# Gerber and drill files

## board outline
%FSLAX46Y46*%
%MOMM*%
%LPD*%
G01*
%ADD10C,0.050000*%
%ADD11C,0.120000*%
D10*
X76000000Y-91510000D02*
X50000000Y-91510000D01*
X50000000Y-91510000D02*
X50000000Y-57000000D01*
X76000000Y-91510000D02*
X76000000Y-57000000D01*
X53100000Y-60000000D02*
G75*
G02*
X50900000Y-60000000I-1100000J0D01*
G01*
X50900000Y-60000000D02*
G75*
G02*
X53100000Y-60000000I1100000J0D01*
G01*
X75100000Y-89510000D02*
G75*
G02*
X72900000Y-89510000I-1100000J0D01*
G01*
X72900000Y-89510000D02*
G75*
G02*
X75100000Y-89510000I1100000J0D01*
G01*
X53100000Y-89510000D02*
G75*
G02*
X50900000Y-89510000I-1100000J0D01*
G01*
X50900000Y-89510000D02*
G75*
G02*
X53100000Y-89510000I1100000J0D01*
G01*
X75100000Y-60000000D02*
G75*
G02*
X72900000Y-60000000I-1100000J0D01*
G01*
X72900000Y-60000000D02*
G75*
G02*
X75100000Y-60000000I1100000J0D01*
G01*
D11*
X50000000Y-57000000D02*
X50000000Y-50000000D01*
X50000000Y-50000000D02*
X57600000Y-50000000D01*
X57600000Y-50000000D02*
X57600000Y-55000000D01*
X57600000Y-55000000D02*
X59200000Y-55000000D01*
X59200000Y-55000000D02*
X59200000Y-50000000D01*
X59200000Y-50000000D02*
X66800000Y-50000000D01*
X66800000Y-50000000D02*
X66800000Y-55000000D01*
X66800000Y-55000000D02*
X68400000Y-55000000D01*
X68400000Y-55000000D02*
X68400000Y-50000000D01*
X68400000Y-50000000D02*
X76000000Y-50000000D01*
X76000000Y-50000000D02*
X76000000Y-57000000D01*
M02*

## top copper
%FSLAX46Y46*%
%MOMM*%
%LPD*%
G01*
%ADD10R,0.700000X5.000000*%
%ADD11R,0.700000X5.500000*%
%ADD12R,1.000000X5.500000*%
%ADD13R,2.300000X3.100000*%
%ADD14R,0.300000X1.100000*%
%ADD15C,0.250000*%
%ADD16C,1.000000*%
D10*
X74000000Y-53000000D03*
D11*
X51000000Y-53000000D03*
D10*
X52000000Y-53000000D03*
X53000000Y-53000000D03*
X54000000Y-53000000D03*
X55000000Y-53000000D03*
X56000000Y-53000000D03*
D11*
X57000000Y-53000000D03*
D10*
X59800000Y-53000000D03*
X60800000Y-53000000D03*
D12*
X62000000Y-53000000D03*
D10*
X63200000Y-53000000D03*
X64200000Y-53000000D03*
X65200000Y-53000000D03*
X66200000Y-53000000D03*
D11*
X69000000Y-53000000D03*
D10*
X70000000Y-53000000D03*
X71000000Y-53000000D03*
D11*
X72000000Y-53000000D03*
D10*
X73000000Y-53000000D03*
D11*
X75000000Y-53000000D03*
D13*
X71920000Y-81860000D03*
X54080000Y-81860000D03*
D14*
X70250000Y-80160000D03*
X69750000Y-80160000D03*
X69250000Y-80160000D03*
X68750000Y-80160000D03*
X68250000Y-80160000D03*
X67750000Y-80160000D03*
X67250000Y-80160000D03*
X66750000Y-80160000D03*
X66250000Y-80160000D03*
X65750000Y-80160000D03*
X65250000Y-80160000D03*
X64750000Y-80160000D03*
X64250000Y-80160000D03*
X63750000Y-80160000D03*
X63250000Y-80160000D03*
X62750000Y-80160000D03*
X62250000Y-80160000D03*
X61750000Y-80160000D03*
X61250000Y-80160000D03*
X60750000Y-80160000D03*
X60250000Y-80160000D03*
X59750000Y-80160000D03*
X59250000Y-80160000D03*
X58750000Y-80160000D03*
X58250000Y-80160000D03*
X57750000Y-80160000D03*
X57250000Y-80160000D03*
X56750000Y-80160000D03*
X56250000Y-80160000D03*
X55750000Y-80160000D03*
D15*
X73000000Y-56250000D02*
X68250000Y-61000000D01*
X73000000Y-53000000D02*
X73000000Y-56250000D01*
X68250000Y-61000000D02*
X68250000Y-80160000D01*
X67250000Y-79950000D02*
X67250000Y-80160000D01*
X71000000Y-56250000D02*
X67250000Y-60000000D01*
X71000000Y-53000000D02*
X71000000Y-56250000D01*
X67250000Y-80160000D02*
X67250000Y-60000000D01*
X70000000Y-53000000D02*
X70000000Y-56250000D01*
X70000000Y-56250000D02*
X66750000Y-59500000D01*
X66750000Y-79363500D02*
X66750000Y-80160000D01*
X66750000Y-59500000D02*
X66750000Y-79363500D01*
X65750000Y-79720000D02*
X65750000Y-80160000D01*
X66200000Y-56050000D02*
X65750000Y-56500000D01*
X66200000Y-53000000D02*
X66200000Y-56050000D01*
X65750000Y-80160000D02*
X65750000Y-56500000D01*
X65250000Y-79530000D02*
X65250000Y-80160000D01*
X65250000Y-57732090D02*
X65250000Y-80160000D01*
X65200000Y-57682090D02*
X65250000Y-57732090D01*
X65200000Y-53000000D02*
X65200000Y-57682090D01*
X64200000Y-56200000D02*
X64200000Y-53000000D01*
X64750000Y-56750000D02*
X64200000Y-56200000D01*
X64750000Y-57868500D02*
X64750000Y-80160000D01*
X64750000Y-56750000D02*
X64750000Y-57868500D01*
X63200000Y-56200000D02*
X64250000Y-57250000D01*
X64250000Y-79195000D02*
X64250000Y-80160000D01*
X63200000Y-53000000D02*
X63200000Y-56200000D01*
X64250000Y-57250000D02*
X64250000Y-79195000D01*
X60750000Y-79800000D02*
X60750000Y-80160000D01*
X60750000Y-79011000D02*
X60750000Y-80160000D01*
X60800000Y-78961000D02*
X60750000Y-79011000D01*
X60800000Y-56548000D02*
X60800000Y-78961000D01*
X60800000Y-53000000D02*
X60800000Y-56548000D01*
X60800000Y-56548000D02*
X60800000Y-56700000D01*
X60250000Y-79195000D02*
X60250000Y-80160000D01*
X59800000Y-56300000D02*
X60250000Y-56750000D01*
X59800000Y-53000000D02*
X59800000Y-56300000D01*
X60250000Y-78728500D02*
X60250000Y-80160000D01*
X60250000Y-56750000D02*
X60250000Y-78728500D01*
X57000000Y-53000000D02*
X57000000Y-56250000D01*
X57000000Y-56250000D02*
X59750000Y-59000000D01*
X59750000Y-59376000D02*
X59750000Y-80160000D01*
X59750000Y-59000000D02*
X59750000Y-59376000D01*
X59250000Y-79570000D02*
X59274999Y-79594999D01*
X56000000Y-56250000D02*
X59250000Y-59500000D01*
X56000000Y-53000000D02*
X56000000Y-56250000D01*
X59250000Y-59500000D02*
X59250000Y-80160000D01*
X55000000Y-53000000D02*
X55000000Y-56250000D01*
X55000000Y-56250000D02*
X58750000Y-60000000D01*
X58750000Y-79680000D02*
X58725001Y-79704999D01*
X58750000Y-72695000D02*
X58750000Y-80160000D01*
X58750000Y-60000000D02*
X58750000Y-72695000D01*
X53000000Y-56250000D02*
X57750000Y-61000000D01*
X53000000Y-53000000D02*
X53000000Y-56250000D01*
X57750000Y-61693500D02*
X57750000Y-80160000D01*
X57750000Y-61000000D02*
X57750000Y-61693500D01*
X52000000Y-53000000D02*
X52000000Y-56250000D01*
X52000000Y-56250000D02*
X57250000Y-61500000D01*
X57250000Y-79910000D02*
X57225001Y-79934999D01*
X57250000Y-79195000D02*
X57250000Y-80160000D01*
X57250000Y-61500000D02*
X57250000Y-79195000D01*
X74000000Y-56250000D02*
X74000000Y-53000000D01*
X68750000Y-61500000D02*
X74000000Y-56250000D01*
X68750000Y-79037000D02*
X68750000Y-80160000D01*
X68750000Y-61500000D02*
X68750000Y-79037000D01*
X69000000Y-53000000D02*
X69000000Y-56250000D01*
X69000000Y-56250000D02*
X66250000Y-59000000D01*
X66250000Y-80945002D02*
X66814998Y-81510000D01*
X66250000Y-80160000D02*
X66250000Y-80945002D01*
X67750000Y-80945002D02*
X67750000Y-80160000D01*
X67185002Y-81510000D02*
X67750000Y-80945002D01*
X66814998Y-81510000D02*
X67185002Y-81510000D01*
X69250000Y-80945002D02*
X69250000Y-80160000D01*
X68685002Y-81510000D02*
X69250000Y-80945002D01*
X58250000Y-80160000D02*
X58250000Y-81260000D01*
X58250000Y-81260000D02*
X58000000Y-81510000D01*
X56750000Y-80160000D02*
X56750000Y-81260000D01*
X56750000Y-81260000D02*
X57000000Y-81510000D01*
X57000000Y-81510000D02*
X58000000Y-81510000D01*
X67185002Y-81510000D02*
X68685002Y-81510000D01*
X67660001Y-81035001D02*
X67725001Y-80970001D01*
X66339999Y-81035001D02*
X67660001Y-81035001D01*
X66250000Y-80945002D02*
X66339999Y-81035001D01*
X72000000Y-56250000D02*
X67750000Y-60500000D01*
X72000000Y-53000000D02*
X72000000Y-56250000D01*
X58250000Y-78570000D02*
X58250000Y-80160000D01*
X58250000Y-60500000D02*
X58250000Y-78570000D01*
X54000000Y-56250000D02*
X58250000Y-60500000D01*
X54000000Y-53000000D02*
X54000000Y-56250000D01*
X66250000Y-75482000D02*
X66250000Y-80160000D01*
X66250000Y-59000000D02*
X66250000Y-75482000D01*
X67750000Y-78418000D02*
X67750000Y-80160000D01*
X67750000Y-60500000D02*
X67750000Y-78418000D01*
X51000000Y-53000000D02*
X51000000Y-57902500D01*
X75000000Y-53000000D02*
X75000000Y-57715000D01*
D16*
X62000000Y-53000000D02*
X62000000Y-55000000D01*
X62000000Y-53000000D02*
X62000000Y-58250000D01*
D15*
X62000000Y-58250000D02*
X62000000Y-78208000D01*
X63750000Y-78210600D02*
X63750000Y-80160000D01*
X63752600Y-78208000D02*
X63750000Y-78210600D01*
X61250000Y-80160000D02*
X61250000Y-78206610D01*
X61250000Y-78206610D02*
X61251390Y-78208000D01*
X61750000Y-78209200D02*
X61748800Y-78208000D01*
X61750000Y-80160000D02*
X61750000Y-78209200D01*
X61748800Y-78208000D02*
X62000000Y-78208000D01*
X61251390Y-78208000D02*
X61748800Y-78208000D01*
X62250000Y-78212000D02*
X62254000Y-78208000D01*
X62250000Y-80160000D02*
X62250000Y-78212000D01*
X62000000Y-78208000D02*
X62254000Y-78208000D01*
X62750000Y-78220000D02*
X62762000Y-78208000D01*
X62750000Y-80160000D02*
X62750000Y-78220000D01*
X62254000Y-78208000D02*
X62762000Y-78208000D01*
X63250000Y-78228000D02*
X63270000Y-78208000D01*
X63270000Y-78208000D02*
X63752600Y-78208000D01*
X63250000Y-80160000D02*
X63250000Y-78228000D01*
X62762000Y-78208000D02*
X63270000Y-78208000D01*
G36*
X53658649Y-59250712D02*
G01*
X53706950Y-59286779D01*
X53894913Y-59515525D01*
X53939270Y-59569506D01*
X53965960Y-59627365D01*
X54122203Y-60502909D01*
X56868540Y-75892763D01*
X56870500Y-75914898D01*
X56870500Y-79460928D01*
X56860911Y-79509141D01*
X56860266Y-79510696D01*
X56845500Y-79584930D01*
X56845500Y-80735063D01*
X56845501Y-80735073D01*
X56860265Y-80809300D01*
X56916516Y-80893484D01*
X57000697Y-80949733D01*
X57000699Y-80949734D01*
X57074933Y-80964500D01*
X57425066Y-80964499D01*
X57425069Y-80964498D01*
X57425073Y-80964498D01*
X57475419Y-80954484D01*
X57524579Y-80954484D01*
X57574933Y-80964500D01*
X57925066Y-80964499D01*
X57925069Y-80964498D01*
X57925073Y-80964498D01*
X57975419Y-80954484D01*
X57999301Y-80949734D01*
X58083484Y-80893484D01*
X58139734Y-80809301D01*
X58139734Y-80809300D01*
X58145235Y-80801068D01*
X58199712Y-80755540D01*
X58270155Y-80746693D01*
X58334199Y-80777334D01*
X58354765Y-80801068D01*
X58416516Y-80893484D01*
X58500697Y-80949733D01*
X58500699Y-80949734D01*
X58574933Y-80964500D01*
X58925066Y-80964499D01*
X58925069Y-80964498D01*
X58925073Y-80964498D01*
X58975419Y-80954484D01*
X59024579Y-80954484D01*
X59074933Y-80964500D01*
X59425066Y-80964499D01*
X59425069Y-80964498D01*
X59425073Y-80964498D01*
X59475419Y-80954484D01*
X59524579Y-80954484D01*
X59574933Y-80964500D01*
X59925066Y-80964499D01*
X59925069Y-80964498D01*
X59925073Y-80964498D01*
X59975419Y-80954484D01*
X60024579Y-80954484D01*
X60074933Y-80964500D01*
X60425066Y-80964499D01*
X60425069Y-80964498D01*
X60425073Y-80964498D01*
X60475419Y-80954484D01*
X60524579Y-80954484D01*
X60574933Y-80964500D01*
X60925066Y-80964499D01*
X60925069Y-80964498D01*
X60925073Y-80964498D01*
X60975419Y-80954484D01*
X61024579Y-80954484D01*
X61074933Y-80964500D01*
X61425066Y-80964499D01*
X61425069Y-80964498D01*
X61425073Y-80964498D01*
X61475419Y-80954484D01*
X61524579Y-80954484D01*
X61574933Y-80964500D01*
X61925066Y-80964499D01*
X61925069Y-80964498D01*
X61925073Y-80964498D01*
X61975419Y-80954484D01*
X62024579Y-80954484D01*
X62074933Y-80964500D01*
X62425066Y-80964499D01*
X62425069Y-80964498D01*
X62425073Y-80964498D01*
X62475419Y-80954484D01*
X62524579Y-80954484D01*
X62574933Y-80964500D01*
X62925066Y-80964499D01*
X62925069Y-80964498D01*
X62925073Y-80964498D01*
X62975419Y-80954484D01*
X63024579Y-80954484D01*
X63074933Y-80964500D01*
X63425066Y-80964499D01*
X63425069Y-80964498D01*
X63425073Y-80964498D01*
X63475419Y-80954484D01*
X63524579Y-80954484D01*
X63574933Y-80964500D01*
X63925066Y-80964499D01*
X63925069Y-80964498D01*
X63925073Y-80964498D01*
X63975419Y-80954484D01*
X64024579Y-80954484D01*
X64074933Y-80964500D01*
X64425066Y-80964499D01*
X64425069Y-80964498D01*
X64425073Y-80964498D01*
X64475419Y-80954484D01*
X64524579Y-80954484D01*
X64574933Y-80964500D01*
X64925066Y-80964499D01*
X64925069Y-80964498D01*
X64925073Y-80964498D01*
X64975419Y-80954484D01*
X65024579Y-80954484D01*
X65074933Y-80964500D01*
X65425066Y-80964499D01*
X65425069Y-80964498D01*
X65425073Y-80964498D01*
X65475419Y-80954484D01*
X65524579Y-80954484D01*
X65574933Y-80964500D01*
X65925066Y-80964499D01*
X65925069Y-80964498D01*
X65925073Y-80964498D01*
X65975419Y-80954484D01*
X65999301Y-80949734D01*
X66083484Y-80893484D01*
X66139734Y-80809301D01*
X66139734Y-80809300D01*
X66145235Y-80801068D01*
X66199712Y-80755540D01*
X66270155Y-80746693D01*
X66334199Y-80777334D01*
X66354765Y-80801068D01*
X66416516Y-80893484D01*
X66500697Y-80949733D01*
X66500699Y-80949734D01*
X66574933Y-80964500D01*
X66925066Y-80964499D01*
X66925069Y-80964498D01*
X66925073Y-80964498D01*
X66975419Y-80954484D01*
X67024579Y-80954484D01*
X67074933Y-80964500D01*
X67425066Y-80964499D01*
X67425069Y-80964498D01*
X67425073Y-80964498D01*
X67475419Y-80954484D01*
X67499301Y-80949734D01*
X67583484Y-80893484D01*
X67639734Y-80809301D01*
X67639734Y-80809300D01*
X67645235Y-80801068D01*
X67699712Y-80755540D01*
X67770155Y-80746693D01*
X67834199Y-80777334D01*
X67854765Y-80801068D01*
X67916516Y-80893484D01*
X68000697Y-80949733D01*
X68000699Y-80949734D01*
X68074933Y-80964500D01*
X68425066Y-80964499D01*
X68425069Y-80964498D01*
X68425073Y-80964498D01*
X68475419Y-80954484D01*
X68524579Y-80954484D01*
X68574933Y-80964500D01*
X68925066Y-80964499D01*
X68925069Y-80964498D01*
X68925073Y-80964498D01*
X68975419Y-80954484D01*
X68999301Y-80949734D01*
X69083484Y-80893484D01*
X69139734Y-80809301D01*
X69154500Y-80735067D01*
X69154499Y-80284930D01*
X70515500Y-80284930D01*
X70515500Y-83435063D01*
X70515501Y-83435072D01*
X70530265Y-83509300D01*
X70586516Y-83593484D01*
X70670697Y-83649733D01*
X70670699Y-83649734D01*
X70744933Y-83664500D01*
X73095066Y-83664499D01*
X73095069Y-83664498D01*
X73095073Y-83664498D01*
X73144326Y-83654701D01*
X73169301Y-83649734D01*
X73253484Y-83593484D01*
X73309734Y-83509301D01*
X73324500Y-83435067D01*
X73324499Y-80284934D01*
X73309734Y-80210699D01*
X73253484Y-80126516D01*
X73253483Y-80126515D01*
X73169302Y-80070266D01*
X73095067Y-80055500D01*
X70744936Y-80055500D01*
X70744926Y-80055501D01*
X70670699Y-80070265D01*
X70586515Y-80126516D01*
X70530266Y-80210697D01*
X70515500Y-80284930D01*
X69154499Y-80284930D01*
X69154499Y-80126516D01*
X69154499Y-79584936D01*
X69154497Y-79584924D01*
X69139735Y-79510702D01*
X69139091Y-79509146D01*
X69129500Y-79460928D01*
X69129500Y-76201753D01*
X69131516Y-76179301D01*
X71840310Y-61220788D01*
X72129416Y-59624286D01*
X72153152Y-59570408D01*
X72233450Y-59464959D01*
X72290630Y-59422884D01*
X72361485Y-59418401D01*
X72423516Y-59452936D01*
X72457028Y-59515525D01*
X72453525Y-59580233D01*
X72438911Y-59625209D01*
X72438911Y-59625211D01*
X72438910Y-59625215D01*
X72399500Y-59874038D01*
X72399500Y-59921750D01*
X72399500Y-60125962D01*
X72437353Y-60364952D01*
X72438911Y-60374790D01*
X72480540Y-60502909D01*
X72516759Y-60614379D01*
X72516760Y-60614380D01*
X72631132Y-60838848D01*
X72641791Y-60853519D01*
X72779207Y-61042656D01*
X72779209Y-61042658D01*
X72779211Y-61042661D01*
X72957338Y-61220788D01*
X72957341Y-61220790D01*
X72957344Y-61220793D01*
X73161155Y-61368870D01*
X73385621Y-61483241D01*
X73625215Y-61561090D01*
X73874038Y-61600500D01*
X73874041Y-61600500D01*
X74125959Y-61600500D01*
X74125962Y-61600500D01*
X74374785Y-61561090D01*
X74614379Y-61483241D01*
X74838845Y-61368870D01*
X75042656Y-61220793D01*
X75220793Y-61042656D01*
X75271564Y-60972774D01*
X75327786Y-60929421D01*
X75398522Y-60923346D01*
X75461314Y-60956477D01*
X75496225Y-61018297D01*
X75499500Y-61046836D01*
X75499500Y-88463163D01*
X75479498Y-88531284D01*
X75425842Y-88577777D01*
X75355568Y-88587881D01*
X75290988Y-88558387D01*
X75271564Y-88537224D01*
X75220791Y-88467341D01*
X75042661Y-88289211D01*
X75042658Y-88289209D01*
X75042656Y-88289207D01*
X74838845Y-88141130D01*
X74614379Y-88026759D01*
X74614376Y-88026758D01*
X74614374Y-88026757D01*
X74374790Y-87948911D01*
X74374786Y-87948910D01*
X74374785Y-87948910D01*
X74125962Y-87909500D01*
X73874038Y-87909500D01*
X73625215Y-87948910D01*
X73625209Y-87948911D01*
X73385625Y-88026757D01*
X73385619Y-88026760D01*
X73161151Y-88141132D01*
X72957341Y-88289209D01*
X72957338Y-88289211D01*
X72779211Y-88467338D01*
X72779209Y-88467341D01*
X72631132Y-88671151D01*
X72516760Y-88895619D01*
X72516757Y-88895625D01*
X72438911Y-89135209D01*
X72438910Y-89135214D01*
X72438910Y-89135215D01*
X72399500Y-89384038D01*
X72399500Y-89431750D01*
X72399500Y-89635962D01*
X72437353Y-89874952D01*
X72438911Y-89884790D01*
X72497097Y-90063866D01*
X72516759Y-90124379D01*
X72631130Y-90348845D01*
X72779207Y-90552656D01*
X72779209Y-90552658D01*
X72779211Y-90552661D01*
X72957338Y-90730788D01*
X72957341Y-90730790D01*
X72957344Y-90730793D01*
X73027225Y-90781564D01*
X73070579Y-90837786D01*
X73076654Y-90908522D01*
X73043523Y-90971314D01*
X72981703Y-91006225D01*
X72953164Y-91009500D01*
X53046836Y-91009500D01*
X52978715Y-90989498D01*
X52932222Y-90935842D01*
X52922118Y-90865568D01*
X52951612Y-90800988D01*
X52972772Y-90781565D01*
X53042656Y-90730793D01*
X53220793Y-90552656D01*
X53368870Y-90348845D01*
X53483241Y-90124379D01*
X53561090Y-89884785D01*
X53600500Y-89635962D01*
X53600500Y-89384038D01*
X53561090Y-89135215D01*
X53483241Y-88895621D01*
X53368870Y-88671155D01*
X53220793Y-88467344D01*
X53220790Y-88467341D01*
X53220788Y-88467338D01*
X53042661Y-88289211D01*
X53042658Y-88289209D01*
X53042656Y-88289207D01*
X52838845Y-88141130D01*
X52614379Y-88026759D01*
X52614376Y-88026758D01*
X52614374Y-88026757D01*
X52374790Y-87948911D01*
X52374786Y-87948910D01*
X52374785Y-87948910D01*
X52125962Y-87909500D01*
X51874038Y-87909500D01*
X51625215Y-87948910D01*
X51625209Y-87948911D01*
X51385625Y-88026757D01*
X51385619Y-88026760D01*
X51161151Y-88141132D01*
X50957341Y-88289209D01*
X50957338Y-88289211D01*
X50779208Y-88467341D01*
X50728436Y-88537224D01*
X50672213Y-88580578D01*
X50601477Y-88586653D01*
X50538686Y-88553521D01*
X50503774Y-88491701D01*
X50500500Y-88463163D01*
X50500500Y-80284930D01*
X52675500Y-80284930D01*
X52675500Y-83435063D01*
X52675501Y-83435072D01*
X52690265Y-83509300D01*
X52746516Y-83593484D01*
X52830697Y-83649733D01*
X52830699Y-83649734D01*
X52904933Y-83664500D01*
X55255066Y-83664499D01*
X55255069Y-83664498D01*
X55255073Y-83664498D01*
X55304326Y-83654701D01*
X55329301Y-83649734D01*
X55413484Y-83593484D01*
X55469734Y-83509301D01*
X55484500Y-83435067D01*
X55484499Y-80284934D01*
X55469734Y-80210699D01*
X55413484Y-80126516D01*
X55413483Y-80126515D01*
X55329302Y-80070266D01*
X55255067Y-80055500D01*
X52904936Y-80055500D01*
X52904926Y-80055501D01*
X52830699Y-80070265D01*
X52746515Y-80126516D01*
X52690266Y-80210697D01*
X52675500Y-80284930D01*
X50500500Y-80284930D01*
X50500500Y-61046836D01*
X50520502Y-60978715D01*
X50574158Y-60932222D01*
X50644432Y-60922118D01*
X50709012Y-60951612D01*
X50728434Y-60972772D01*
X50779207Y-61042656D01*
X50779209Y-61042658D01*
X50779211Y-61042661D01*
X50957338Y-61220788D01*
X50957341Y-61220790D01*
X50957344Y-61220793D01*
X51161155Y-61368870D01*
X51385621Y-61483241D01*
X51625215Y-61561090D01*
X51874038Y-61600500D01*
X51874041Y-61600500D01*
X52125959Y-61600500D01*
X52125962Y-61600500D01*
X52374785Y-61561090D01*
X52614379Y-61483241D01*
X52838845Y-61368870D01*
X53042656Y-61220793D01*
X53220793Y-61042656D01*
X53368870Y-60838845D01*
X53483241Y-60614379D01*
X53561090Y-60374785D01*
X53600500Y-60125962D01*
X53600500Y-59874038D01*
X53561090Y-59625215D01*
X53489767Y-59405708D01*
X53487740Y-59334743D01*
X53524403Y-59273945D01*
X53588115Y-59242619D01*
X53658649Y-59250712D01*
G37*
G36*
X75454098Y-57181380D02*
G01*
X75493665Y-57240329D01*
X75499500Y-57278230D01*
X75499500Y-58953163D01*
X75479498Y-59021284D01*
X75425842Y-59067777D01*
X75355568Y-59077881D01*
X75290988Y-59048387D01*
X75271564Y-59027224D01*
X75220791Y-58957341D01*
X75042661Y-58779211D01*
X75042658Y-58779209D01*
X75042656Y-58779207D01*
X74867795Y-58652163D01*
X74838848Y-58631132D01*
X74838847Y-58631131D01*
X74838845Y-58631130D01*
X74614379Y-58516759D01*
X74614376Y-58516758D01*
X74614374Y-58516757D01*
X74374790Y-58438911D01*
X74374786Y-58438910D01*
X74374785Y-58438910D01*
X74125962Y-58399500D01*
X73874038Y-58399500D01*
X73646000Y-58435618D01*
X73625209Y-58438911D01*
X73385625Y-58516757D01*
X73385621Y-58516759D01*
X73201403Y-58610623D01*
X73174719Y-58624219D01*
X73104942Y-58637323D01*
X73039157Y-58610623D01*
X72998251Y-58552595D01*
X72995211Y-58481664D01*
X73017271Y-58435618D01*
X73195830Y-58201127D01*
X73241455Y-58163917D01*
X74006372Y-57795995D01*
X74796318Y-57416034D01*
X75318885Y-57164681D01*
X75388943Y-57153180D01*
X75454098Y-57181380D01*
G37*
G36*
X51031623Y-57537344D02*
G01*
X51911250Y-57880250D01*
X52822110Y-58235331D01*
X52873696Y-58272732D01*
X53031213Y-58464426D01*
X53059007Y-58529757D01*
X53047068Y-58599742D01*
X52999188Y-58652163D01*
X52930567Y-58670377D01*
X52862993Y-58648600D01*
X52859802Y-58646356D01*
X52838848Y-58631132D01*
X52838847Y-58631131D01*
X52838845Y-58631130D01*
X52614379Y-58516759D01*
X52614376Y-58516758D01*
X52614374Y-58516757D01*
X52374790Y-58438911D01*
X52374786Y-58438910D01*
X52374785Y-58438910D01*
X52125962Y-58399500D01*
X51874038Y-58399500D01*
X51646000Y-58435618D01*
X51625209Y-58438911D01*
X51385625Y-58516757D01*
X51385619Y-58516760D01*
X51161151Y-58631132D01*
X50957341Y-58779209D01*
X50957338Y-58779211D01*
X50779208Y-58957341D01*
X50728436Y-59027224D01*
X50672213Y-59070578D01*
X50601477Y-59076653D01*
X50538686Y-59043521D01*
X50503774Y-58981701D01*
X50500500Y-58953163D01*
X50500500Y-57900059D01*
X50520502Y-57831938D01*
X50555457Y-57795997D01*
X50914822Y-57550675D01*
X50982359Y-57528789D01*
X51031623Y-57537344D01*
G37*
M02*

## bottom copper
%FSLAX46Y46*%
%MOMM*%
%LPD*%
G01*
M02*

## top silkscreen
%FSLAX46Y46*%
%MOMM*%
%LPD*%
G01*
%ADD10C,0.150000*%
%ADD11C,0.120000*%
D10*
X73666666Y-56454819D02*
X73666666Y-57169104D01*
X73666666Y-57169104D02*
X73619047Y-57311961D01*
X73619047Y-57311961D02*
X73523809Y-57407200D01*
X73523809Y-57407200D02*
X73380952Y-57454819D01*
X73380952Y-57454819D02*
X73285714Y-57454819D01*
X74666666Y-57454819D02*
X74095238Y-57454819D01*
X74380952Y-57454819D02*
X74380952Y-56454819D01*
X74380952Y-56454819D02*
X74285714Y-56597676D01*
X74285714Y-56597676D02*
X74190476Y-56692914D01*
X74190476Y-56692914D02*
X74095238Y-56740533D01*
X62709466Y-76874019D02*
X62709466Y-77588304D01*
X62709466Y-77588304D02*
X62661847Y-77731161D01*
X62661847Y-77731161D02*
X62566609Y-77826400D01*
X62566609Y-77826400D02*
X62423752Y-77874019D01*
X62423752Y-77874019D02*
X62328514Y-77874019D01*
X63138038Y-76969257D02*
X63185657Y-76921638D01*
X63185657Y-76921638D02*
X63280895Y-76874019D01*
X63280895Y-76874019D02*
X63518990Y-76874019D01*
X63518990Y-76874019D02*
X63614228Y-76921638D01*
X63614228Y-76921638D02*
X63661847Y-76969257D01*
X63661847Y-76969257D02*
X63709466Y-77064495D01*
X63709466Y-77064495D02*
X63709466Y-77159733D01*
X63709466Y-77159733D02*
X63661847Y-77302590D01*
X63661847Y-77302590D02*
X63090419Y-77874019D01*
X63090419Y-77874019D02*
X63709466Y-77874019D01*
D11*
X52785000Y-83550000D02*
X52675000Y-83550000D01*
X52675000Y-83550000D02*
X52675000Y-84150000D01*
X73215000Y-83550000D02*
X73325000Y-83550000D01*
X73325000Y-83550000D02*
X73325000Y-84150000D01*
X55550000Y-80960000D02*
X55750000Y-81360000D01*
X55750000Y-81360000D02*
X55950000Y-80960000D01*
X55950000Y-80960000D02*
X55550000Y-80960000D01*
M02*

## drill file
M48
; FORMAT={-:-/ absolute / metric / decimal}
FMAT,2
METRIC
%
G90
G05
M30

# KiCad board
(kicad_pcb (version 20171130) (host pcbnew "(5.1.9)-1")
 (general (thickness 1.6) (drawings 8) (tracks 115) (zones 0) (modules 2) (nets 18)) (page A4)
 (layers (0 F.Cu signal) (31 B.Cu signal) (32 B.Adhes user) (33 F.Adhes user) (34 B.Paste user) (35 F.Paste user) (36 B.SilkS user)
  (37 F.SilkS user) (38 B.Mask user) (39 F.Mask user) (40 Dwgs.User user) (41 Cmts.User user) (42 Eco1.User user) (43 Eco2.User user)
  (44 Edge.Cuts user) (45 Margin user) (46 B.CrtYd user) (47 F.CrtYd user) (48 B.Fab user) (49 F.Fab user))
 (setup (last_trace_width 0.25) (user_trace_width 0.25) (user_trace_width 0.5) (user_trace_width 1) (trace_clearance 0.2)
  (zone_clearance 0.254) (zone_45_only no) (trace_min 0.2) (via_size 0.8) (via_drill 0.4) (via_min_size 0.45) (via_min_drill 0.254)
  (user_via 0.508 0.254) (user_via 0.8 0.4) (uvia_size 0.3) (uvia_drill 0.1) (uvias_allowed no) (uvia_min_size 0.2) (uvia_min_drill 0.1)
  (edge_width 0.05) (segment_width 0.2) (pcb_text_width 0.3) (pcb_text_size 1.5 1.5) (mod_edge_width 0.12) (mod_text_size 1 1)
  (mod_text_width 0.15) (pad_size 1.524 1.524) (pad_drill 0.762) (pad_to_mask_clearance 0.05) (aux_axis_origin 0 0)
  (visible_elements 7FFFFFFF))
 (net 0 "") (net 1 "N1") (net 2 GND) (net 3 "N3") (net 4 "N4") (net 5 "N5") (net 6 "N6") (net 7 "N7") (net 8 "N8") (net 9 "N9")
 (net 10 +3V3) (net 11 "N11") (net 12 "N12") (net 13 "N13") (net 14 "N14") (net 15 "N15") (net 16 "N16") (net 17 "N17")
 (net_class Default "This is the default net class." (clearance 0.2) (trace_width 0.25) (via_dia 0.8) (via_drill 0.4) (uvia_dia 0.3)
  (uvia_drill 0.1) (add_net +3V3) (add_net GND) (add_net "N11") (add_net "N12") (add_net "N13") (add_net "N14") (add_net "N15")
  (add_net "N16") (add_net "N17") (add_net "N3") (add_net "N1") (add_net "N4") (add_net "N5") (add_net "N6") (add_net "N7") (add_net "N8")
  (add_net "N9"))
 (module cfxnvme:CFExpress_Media (layer F.Cu) (at 49 48)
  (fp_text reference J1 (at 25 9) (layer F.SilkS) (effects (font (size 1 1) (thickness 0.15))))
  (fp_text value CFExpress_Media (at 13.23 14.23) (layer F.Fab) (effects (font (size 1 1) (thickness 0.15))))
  (fp_line (start 1 9) (end 1 2) (layer Edge.Cuts) (width 0.12))
  (fp_line (start 1 2) (end 8.6 2) (layer Edge.Cuts) (width 0.12))
  (fp_line (start 8.6 2) (end 8.6 7) (layer Edge.Cuts) (width 0.12))
  (fp_line (start 8.6 7) (end 10.2 7) (layer Edge.Cuts) (width 0.12))
  (fp_line (start 10.2 7) (end 10.2 2) (layer Edge.Cuts) (width 0.12))
  (fp_line (start 10.2 2) (end 17.8 2) (layer Edge.Cuts) (width 0.12))
  (fp_line (start 17.8 2) (end 17.8 7) (layer Edge.Cuts) (width 0.12))
  (fp_line (start 17.8 7) (end 19.4 7) (layer Edge.Cuts) (width 0.12))
  (fp_line (start 19.4 7) (end 19.4 2) (layer Edge.Cuts) (width 0.12))
  (fp_line (start 19.4 2) (end 27 2) (layer Edge.Cuts) (width 0.12))
  (fp_line (start 27 2) (end 27 9) (layer Edge.Cuts) (width 0.12))
  (pad 20 connect rect (at 25 5) (size 0.7 5) (layers F.Cu F.Mask) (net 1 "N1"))
  (pad 1 connect rect (at 2 5) (size 0.7 5.5) (layers F.Cu F.Mask) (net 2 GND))
  (pad 2 connect rect (at 3 5) (size 0.7 5) (layers F.Cu F.Mask) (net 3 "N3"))
  (pad 3 connect rect (at 4 5) (size 0.7 5) (layers F.Cu F.Mask) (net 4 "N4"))
  (pad 4 connect rect (at 5 5) (size 0.7 5) (layers F.Cu F.Mask) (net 2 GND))
  (pad 5 connect rect (at 6 5) (size 0.7 5) (layers F.Cu F.Mask) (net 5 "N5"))
  (pad 6 connect rect (at 7 5) (size 0.7 5) (layers F.Cu F.Mask) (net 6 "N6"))
  (pad 7 connect rect (at 8 5) (size 0.7 5.5) (layers F.Cu F.Mask) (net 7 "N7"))
  (pad 8 connect rect (at 10.8 5) (size 0.7 5) (layers F.Cu F.Mask) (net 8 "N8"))
  (pad 9 connect rect (at 11.8 5) (size 0.7 5) (layers F.Cu F.Mask) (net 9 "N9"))
  (pad 10 connect rect (at 13 5) (size 1 5.5) (layers F.Cu F.Mask) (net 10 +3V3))
  (pad 11 connect rect (at 14.2 5) (size 0.7 5) (layers F.Cu F.Mask) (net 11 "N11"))
  (pad 12 connect rect (at 15.2 5) (size 0.7 5) (layers F.Cu F.Mask) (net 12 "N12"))
  (pad 13 connect rect (at 16.2 5) (size 0.7 5) (layers F.Cu F.Mask) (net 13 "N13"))
  (pad 14 connect rect (at 17.2 5) (size 0.7 5) (layers F.Cu F.Mask) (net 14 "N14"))
  (pad 15 connect rect (at 20 5) (size 0.7 5.5) (layers F.Cu F.Mask) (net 2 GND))
  (pad 16 connect rect (at 21 5) (size 0.7 5) (layers F.Cu F.Mask) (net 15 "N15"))
  (pad 17 connect rect (at 22 5) (size 0.7 5) (layers F.Cu F.Mask) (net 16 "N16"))
  (pad 18 connect rect (at 23 5) (size 0.7 5.5) (layers F.Cu F.Mask) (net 2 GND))
  (pad 19 connect rect (at 24 5) (size 0.7 5) (layers F.Cu F.Mask) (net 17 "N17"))
  (pad 21 connect rect (at 26 5) (size 0.7 5.5) (layers F.Cu F.Mask) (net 2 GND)))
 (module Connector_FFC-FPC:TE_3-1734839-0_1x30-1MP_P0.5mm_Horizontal (layer F.Cu) (at 63 81.51)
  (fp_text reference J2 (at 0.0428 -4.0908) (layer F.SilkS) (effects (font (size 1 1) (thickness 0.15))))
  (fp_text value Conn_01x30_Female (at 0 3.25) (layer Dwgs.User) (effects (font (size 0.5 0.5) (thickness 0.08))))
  (fp_line (start -10.215 2.04) (end -10.325 2.04) (layer F.SilkS) (width 0.12))
  (fp_line (start -10.325 2.04) (end -10.325 2.64) (layer F.SilkS) (width 0.12))
  (fp_line (start 10.215 2.04) (end 10.325 2.04) (layer F.SilkS) (width 0.12))
  (fp_line (start 10.325 2.04) (end 10.325 2.64) (layer F.SilkS) (width 0.12))
  (fp_line (start -7.45 -0.55) (end -7.25 -0.15) (layer F.SilkS) (width 0.12))
  (fp_line (start -7.25 -0.15) (end -7.05 -0.55) (layer F.SilkS) (width 0.12))
  (fp_line (start -7.05 -0.55) (end -7.45 -0.55) (layer F.SilkS) (width 0.12))
  (pad MP smd rect (at 8.92 0.35) (size 2.3 3.1) (layers F.Cu F.Paste F.Mask))
  (pad MP smd rect (at -8.92 0.35) (size 2.3 3.1) (layers F.Cu F.Paste F.Mask))
  (pad 30 smd rect (at 7.25 -1.35) (size 0.3 1.1) (layers F.Cu F.Paste F.Mask) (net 2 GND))
  (pad 29 smd rect (at 6.75 -1.35) (size 0.3 1.1) (layers F.Cu F.Paste F.Mask) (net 2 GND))
  (pad 28 smd rect (at 6.25 -1.35) (size 0.3 1.1) (layers F.Cu F.Paste F.Mask) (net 2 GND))
  (pad 27 smd rect (at 5.75 -1.35) (size 0.3 1.1) (layers F.Cu F.Paste F.Mask) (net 1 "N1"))
  (pad 26 smd rect (at 5.25 -1.35) (size 0.3 1.1) (layers F.Cu F.Paste F.Mask) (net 17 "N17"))
  (pad 25 smd rect (at 4.75 -1.35) (size 0.3 1.1) (layers F.Cu F.Paste F.Mask) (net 2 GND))
  (pad 24 smd rect (at 4.25 -1.35) (size 0.3 1.1) (layers F.Cu F.Paste F.Mask) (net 16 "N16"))
  (pad 23 smd rect (at 3.75 -1.35) (size 0.3 1.1) (layers F.Cu F.Paste F.Mask) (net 15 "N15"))
  (pad 22 smd rect (at 3.25 -1.35) (size 0.3 1.1) (layers F.Cu F.Paste F.Mask) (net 2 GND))
  (pad 21 smd rect (at 2.75 -1.35) (size 0.3 1.1) (layers F.Cu F.Paste F.Mask) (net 14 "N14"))
  (pad 20 smd rect (at 2.25 -1.35) (size 0.3 1.1) (layers F.Cu F.Paste F.Mask) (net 13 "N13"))
  (pad 19 smd rect (at 1.75 -1.35) (size 0.3 1.1) (layers F.Cu F.Paste F.Mask) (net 12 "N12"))
  (pad 18 smd rect (at 1.25 -1.35) (size 0.3 1.1) (layers F.Cu F.Paste F.Mask) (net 11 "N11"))
  (pad 17 smd rect (at 0.75 -1.35) (size 0.3 1.1) (layers F.Cu F.Paste F.Mask) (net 10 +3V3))
  (pad 16 smd rect (at 0.25 -1.35) (size 0.3 1.1) (layers F.Cu F.Paste F.Mask) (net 10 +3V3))
  (pad 15 smd rect (at -0.25 -1.35) (size 0.3 1.1) (layers F.Cu F.Paste F.Mask) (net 10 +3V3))
  (pad 14 smd rect (at -0.75 -1.35) (size 0.3 1.1) (layers F.Cu F.Paste F.Mask) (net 10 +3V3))
  (pad 13 smd rect (at -1.25 -1.35) (size 0.3 1.1) (layers F.Cu F.Paste F.Mask) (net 10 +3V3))
  (pad 12 smd rect (at -1.75 -1.35) (size 0.3 1.1) (layers F.Cu F.Paste F.Mask) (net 10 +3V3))
  (pad 11 smd rect (at -2.25 -1.35) (size 0.3 1.1) (layers F.Cu F.Paste F.Mask) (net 9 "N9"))
  (pad 10 smd rect (at -2.75 -1.35) (size 0.3 1.1) (layers F.Cu F.Paste F.Mask) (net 8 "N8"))
  (pad 9 smd rect (at -3.25 -1.35) (size 0.3 1.1) (layers F.Cu F.Paste F.Mask) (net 7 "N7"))
  (pad 8 smd rect (at -3.75 -1.35) (size 0.3 1.1) (layers F.Cu F.Paste F.Mask) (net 6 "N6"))
  (pad 7 smd rect (at -4.25 -1.35) (size 0.3 1.1) (layers F.Cu F.Paste F.Mask) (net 5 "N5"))
  (pad 6 smd rect (at -4.75 -1.35) (size 0.3 1.1) (layers F.Cu F.Paste F.Mask) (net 2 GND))
  (pad 5 smd rect (at -5.25 -1.35) (size 0.3 1.1) (layers F.Cu F.Paste F.Mask) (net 4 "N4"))
  (pad 4 smd rect (at -5.75 -1.35) (size 0.3 1.1) (layers F.Cu F.Paste F.Mask) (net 3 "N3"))
  (pad 3 smd rect (at -6.25 -1.35) (size 0.3 1.1) (layers F.Cu F.Paste F.Mask) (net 2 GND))
  (pad 2 smd rect (at -6.75 -1.35) (size 0.3 1.1) (layers F.Cu F.Paste F.Mask) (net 2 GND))
  (pad 1 smd rect (at -7.25 -1.35) (size 0.3 1.1) (layers F.Cu F.Paste F.Mask) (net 2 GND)))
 (gr_line (start 76 91.51) (end 50 91.51) (layer Edge.Cuts) (width 0.05))
 (gr_line (start 50 91.51) (end 50 57) (layer Edge.Cuts) (width 0.05))
 (gr_line (start 76 91.51) (end 76 57) (layer Edge.Cuts) (width 0.05))
 (gr_circle (center 52 60) (end 53.1 60) (layer Edge.Cuts) (width 0.05))
 (gr_circle (center 74 89.51) (end 75.1 89.51) (layer Edge.Cuts) (width 0.05))
 (gr_circle (center 52 89.51) (end 53.1 89.51) (layer Edge.Cuts) (width 0.05))
 (gr_circle (center 74 60) (end 75.1 60) (layer Edge.Cuts) (width 0.05))
 (segment (start 73 56.25) (end 68.25 61) (width 0.25) (layer F.Cu) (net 17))
 (segment (start 73 53) (end 73 56.25) (width 0.25) (layer F.Cu) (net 17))
 (segment (start 68.25 61) (end 68.25 80.16) (width 0.25) (layer F.Cu) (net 17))
 (segment (start 67.25 79.95) (end 67.25 80.16) (width 0.25) (layer F.Cu) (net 16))
 (segment (start 71 56.25) (end 67.25 60) (width 0.25) (layer F.Cu) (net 16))
 (segment (start 71 53) (end 71 56.25) (width 0.25) (layer F.Cu) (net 16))
 (segment (start 67.25 80.16) (end 67.25 60) (width 0.25) (layer F.Cu) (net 16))
 (segment (start 70 53) (end 70 56.25) (width 0.25) (layer F.Cu) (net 15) (status 400000))
 (segment (start 70 56.25) (end 66.75 59.5) (width 0.25) (layer F.Cu) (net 15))
 (segment (start 66.75 79.3635) (end 66.75 80.16) (width 0.25) (layer F.Cu) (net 15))
 (segment (start 66.75 59.5) (end 66.75 79.3635) (width 0.25) (layer F.Cu) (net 15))
 (segment (start 65.75 79.72) (end 65.75 80.16) (width 0.25) (layer F.Cu) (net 14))
 (segment (start 66.2 56.05) (end 65.75 56.5) (width 0.25) (layer F.Cu) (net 14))
 (segment (start 66.2 53) (end 66.2 56.05) (width 0.25) (layer F.Cu) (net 14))
 (segment (start 65.75 80.16) (end 65.75 56.5) (width 0.25) (layer F.Cu) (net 14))
 (segment (start 65.25 79.53) (end 65.25 80.16) (width 0.25) (layer F.Cu) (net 13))
 (segment (start 65.25 57.73209) (end 65.25 80.16) (width 0.25) (layer F.Cu) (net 13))
 (segment (start 65.2 57.68209) (end 65.25 57.73209) (width 0.25) (layer F.Cu) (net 13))
 (segment (start 65.2 53) (end 65.2 57.68209) (width 0.25) (layer F.Cu) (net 13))
 (segment (start 64.2 56.2) (end 64.2 53) (width 0.25) (layer F.Cu) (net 12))
 (segment (start 64.75 56.75) (end 64.2 56.2) (width 0.25) (layer F.Cu) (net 12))
 (segment (start 64.75 57.8685) (end 64.75 80.16) (width 0.25) (layer F.Cu) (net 12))
 (segment (start 64.75 56.75) (end 64.75 57.8685) (width 0.25) (layer F.Cu) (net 12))
 (segment (start 63.2 56.2) (end 64.25 57.25) (width 0.25) (layer F.Cu) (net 11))
 (segment (start 64.25 79.195) (end 64.25 80.16) (width 0.25) (layer F.Cu) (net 11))
 (segment (start 63.2 53) (end 63.2 56.2) (width 0.25) (layer F.Cu) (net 11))
 (segment (start 64.25 57.25) (end 64.25 79.195) (width 0.25) (layer F.Cu) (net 11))
 (segment (start 60.75 79.8) (end 60.75 80.16) (width 0.25) (layer F.Cu) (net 9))
 (segment (start 60.75 79.011) (end 60.75 80.16) (width 0.25) (layer F.Cu) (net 9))
 (segment (start 60.8 78.961) (end 60.75 79.011) (width 0.25) (layer F.Cu) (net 9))
 (segment (start 60.8 56.548) (end 60.8 78.961) (width 0.25) (layer F.Cu) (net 9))
 (segment (start 60.8 53) (end 60.8 56.548) (width 0.25) (layer F.Cu) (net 9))
 (segment (start 60.8 56.548) (end 60.8 56.7) (width 0.25) (layer F.Cu) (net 9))
 (segment (start 60.25 79.195) (end 60.25 80.16) (width 0.25) (layer F.Cu) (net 8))
 (segment (start 59.8 56.3) (end 60.25 56.75) (width 0.25) (layer F.Cu) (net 8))
 (segment (start 59.8 53) (end 59.8 56.3) (width 0.25) (layer F.Cu) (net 8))
 (segment (start 60.25 78.7285) (end 60.25 80.16) (width 0.25) (layer F.Cu) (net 8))
 (segment (start 60.25 56.75) (end 60.25 78.7285) (width 0.25) (layer F.Cu) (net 8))
 (segment (start 57 53) (end 57 56.25) (width 0.25) (layer F.Cu) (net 7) (status 400000))
 (segment (start 57 56.25) (end 59.75 59) (width 0.25) (layer F.Cu) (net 7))
 (segment (start 59.75 59.376) (end 59.75 80.16) (width 0.25) (layer F.Cu) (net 7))
 (segment (start 59.75 59) (end 59.75 59.376) (width 0.25) (layer F.Cu) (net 7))
 (segment (start 59.25 79.57) (end 59.274999 79.594999) (width 0.25) (layer F.Cu) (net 6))
 (segment (start 56 56.25) (end 59.25 59.5) (width 0.25) (layer F.Cu) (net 6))
 (segment (start 56 53) (end 56 56.25) (width 0.25) (layer F.Cu) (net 6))
 (segment (start 59.25 59.5) (end 59.25 80.16) (width 0.25) (layer F.Cu) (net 6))
 (segment (start 55 53) (end 55 56.25) (width 0.25) (layer F.Cu) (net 5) (status 400000))
 (segment (start 55 56.25) (end 58.75 60) (width 0.25) (layer F.Cu) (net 5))
 (segment (start 58.75 79.68) (end 58.725001 79.704999) (width 0.25) (layer F.Cu) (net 5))
 (segment (start 58.75 72.695) (end 58.75 80.16) (width 0.25) (layer F.Cu) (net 5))
 (segment (start 58.75 60) (end 58.75 72.695) (width 0.25) (layer F.Cu) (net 5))
 (segment (start 53 56.25) (end 57.75 61) (width 0.25) (layer F.Cu) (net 4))
 (segment (start 53 53) (end 53 56.25) (width 0.25) (layer F.Cu) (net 4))
 (segment (start 57.75 61.6935) (end 57.75 80.16) (width 0.25) (layer F.Cu) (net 4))
 (segment (start 57.75 61) (end 57.75 61.6935) (width 0.25) (layer F.Cu) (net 4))
 (segment (start 52 53) (end 52 56.25) (width 0.25) (layer F.Cu) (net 3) (status 400000))
 (segment (start 52 56.25) (end 57.25 61.5) (width 0.25) (layer F.Cu) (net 3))
 (segment (start 57.25 79.91) (end 57.225001 79.934999) (width 0.25) (layer F.Cu) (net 3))
 (segment (start 57.25 79.195) (end 57.25 80.16) (width 0.25) (layer F.Cu) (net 3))
 (segment (start 57.25 61.5) (end 57.25 79.195) (width 0.25) (layer F.Cu) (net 3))
 (segment (start 74 56.25) (end 74 53) (width 0.25) (layer F.Cu) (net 1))
 (segment (start 68.75 61.5) (end 74 56.25) (width 0.25) (layer F.Cu) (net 1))
 (segment (start 68.75 79.037) (end 68.75 80.16) (width 0.25) (layer F.Cu) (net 1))
 (segment (start 68.75 61.5) (end 68.75 79.037) (width 0.25) (layer F.Cu) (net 1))
 (segment (start 69 53) (end 69 56.25) (width 0.25) (layer F.Cu) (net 2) (status 400000))
 (segment (start 69 56.25) (end 66.25 59) (width 0.25) (layer F.Cu) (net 2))
 (segment (start 66.25 80.945002) (end 66.814998 81.51) (width 0.25) (layer F.Cu) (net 2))
 (segment (start 66.25 80.16) (end 66.25 80.945002) (width 0.25) (layer F.Cu) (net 2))
 (segment (start 67.75 80.945002) (end 67.75 80.16) (width 0.25) (layer F.Cu) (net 2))
 (segment (start 67.185002 81.51) (end 67.75 80.945002) (width 0.25) (layer F.Cu) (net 2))
 (segment (start 66.814998 81.51) (end 67.185002 81.51) (width 0.25) (layer F.Cu) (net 2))
 (segment (start 69.25 80.945002) (end 69.25 80.16) (width 0.25) (layer F.Cu) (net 2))
 (segment (start 68.685002 81.51) (end 69.25 80.945002) (width 0.25) (layer F.Cu) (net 2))
 (segment (start 58.25 80.16) (end 58.25 81.26) (width 0.25) (layer F.Cu) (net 2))
 (segment (start 58.25 81.26) (end 58 81.51) (width 0.25) (layer F.Cu) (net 2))
 (segment (start 56.75 80.16) (end 56.75 81.26) (width 0.25) (layer F.Cu) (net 2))
 (segment (start 56.75 81.26) (end 57 81.51) (width 0.25) (layer F.Cu) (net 2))
 (segment (start 57 81.51) (end 58 81.51) (width 0.25) (layer F.Cu) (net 2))
 (segment (start 67.185002 81.51) (end 68.685002 81.51) (width 0.25) (layer F.Cu) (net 2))
 (segment (start 67.660001 81.035001) (end 67.725001 80.970001) (width 0.25) (layer F.Cu) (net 2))
 (segment (start 66.339999 81.035001) (end 67.660001 81.035001) (width 0.25) (layer F.Cu) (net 2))
 (segment (start 66.25 80.945002) (end 66.339999 81.035001) (width 0.25) (layer F.Cu) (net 2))
 (segment (start 72 56.25) (end 67.75 60.5) (width 0.25) (layer F.Cu) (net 2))
 (segment (start 72 53) (end 72 56.25) (width 0.25) (layer F.Cu) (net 2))
 (segment (start 58.25 78.57) (end 58.25 80.16) (width 0.25) (layer F.Cu) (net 2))
 (segment (start 58.25 60.5) (end 58.25 78.57) (width 0.25) (layer F.Cu) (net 2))
 (segment (start 54 56.25) (end 58.25 60.5) (width 0.25) (layer F.Cu) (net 2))
 (segment (start 54 53) (end 54 56.25) (width 0.25) (layer F.Cu) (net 2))
 (segment (start 66.25 75.482) (end 66.25 80.16) (width 0.25) (layer F.Cu) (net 2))
 (segment (start 66.25 59) (end 66.25 75.482) (width 0.25) (layer F.Cu) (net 2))
 (segment (start 67.75 78.418) (end 67.75 80.16) (width 0.25) (layer F.Cu) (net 2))
 (segment (start 67.75 60.5) (end 67.75 78.418) (width 0.25) (layer F.Cu) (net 2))
 (segment (start 51 53) (end 51 57.9025) (width 0.25) (layer F.Cu) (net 2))
 (segment (start 75 53) (end 75 57.715) (width 0.25) (layer F.Cu) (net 2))
 (segment (start 62 53) (end 62 55) (width 1) (layer F.Cu) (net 10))
 (segment (start 62 53) (end 62 58.25) (width 1) (layer F.Cu) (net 10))
 (segment (start 62 58.25) (end 62 78.208) (width 0.25) (layer F.Cu) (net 10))
 (segment (start 63.75 78.2106) (end 63.75 80.16) (width 0.25) (layer F.Cu) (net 10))
 (segment (start 63.7526 78.208) (end 63.75 78.2106) (width 0.25) (layer F.Cu) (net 10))
 (segment (start 61.25 80.16) (end 61.25 78.20661) (width 0.25) (layer F.Cu) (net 10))
 (segment (start 61.25 78.20661) (end 61.25139 78.208) (width 0.25) (layer F.Cu) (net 10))
 (segment (start 61.75 78.2092) (end 61.7488 78.208) (width 0.25) (layer F.Cu) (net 10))
 (segment (start 61.75 80.16) (end 61.75 78.2092) (width 0.25) (layer F.Cu) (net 10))
 (segment (start 61.7488 78.208) (end 62 78.208) (width 0.25) (layer F.Cu) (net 10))
 (segment (start 61.25139 78.208) (end 61.7488 78.208) (width 0.25) (layer F.Cu) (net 10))
 (segment (start 62.25 78.212) (end 62.254 78.208) (width 0.25) (layer F.Cu) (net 10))
 (segment (start 62.25 80.16) (end 62.25 78.212) (width 0.25) (layer F.Cu) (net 10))
 (segment (start 62 78.208) (end 62.254 78.208) (width 0.25) (layer F.Cu) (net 10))
 (segment (start 62.75 78.22) (end 62.762 78.208) (width 0.25) (layer F.Cu) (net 10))
 (segment (start 62.75 80.16) (end 62.75 78.22) (width 0.25) (layer F.Cu) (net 10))
 (segment (start 62.254 78.208) (end 62.762 78.208) (width 0.25) (layer F.Cu) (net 10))
 (segment (start 63.25 78.228) (end 63.27 78.208) (width 0.25) (layer F.Cu) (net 10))
 (segment (start 63.27 78.208) (end 63.7526 78.208) (width 0.25) (layer F.Cu) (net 10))
 (segment (start 63.25 80.16) (end 63.25 78.228) (width 0.25) (layer F.Cu) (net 10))
 (segment (start 62.762 78.208) (end 63.27 78.208) (width 0.25) (layer F.Cu) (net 10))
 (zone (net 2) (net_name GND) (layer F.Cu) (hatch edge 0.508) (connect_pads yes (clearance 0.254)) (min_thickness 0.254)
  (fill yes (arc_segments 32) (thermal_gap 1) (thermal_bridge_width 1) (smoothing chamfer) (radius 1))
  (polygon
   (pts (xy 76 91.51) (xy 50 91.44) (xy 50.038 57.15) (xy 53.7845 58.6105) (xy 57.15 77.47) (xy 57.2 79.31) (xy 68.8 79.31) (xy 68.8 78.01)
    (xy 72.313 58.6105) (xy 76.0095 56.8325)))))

